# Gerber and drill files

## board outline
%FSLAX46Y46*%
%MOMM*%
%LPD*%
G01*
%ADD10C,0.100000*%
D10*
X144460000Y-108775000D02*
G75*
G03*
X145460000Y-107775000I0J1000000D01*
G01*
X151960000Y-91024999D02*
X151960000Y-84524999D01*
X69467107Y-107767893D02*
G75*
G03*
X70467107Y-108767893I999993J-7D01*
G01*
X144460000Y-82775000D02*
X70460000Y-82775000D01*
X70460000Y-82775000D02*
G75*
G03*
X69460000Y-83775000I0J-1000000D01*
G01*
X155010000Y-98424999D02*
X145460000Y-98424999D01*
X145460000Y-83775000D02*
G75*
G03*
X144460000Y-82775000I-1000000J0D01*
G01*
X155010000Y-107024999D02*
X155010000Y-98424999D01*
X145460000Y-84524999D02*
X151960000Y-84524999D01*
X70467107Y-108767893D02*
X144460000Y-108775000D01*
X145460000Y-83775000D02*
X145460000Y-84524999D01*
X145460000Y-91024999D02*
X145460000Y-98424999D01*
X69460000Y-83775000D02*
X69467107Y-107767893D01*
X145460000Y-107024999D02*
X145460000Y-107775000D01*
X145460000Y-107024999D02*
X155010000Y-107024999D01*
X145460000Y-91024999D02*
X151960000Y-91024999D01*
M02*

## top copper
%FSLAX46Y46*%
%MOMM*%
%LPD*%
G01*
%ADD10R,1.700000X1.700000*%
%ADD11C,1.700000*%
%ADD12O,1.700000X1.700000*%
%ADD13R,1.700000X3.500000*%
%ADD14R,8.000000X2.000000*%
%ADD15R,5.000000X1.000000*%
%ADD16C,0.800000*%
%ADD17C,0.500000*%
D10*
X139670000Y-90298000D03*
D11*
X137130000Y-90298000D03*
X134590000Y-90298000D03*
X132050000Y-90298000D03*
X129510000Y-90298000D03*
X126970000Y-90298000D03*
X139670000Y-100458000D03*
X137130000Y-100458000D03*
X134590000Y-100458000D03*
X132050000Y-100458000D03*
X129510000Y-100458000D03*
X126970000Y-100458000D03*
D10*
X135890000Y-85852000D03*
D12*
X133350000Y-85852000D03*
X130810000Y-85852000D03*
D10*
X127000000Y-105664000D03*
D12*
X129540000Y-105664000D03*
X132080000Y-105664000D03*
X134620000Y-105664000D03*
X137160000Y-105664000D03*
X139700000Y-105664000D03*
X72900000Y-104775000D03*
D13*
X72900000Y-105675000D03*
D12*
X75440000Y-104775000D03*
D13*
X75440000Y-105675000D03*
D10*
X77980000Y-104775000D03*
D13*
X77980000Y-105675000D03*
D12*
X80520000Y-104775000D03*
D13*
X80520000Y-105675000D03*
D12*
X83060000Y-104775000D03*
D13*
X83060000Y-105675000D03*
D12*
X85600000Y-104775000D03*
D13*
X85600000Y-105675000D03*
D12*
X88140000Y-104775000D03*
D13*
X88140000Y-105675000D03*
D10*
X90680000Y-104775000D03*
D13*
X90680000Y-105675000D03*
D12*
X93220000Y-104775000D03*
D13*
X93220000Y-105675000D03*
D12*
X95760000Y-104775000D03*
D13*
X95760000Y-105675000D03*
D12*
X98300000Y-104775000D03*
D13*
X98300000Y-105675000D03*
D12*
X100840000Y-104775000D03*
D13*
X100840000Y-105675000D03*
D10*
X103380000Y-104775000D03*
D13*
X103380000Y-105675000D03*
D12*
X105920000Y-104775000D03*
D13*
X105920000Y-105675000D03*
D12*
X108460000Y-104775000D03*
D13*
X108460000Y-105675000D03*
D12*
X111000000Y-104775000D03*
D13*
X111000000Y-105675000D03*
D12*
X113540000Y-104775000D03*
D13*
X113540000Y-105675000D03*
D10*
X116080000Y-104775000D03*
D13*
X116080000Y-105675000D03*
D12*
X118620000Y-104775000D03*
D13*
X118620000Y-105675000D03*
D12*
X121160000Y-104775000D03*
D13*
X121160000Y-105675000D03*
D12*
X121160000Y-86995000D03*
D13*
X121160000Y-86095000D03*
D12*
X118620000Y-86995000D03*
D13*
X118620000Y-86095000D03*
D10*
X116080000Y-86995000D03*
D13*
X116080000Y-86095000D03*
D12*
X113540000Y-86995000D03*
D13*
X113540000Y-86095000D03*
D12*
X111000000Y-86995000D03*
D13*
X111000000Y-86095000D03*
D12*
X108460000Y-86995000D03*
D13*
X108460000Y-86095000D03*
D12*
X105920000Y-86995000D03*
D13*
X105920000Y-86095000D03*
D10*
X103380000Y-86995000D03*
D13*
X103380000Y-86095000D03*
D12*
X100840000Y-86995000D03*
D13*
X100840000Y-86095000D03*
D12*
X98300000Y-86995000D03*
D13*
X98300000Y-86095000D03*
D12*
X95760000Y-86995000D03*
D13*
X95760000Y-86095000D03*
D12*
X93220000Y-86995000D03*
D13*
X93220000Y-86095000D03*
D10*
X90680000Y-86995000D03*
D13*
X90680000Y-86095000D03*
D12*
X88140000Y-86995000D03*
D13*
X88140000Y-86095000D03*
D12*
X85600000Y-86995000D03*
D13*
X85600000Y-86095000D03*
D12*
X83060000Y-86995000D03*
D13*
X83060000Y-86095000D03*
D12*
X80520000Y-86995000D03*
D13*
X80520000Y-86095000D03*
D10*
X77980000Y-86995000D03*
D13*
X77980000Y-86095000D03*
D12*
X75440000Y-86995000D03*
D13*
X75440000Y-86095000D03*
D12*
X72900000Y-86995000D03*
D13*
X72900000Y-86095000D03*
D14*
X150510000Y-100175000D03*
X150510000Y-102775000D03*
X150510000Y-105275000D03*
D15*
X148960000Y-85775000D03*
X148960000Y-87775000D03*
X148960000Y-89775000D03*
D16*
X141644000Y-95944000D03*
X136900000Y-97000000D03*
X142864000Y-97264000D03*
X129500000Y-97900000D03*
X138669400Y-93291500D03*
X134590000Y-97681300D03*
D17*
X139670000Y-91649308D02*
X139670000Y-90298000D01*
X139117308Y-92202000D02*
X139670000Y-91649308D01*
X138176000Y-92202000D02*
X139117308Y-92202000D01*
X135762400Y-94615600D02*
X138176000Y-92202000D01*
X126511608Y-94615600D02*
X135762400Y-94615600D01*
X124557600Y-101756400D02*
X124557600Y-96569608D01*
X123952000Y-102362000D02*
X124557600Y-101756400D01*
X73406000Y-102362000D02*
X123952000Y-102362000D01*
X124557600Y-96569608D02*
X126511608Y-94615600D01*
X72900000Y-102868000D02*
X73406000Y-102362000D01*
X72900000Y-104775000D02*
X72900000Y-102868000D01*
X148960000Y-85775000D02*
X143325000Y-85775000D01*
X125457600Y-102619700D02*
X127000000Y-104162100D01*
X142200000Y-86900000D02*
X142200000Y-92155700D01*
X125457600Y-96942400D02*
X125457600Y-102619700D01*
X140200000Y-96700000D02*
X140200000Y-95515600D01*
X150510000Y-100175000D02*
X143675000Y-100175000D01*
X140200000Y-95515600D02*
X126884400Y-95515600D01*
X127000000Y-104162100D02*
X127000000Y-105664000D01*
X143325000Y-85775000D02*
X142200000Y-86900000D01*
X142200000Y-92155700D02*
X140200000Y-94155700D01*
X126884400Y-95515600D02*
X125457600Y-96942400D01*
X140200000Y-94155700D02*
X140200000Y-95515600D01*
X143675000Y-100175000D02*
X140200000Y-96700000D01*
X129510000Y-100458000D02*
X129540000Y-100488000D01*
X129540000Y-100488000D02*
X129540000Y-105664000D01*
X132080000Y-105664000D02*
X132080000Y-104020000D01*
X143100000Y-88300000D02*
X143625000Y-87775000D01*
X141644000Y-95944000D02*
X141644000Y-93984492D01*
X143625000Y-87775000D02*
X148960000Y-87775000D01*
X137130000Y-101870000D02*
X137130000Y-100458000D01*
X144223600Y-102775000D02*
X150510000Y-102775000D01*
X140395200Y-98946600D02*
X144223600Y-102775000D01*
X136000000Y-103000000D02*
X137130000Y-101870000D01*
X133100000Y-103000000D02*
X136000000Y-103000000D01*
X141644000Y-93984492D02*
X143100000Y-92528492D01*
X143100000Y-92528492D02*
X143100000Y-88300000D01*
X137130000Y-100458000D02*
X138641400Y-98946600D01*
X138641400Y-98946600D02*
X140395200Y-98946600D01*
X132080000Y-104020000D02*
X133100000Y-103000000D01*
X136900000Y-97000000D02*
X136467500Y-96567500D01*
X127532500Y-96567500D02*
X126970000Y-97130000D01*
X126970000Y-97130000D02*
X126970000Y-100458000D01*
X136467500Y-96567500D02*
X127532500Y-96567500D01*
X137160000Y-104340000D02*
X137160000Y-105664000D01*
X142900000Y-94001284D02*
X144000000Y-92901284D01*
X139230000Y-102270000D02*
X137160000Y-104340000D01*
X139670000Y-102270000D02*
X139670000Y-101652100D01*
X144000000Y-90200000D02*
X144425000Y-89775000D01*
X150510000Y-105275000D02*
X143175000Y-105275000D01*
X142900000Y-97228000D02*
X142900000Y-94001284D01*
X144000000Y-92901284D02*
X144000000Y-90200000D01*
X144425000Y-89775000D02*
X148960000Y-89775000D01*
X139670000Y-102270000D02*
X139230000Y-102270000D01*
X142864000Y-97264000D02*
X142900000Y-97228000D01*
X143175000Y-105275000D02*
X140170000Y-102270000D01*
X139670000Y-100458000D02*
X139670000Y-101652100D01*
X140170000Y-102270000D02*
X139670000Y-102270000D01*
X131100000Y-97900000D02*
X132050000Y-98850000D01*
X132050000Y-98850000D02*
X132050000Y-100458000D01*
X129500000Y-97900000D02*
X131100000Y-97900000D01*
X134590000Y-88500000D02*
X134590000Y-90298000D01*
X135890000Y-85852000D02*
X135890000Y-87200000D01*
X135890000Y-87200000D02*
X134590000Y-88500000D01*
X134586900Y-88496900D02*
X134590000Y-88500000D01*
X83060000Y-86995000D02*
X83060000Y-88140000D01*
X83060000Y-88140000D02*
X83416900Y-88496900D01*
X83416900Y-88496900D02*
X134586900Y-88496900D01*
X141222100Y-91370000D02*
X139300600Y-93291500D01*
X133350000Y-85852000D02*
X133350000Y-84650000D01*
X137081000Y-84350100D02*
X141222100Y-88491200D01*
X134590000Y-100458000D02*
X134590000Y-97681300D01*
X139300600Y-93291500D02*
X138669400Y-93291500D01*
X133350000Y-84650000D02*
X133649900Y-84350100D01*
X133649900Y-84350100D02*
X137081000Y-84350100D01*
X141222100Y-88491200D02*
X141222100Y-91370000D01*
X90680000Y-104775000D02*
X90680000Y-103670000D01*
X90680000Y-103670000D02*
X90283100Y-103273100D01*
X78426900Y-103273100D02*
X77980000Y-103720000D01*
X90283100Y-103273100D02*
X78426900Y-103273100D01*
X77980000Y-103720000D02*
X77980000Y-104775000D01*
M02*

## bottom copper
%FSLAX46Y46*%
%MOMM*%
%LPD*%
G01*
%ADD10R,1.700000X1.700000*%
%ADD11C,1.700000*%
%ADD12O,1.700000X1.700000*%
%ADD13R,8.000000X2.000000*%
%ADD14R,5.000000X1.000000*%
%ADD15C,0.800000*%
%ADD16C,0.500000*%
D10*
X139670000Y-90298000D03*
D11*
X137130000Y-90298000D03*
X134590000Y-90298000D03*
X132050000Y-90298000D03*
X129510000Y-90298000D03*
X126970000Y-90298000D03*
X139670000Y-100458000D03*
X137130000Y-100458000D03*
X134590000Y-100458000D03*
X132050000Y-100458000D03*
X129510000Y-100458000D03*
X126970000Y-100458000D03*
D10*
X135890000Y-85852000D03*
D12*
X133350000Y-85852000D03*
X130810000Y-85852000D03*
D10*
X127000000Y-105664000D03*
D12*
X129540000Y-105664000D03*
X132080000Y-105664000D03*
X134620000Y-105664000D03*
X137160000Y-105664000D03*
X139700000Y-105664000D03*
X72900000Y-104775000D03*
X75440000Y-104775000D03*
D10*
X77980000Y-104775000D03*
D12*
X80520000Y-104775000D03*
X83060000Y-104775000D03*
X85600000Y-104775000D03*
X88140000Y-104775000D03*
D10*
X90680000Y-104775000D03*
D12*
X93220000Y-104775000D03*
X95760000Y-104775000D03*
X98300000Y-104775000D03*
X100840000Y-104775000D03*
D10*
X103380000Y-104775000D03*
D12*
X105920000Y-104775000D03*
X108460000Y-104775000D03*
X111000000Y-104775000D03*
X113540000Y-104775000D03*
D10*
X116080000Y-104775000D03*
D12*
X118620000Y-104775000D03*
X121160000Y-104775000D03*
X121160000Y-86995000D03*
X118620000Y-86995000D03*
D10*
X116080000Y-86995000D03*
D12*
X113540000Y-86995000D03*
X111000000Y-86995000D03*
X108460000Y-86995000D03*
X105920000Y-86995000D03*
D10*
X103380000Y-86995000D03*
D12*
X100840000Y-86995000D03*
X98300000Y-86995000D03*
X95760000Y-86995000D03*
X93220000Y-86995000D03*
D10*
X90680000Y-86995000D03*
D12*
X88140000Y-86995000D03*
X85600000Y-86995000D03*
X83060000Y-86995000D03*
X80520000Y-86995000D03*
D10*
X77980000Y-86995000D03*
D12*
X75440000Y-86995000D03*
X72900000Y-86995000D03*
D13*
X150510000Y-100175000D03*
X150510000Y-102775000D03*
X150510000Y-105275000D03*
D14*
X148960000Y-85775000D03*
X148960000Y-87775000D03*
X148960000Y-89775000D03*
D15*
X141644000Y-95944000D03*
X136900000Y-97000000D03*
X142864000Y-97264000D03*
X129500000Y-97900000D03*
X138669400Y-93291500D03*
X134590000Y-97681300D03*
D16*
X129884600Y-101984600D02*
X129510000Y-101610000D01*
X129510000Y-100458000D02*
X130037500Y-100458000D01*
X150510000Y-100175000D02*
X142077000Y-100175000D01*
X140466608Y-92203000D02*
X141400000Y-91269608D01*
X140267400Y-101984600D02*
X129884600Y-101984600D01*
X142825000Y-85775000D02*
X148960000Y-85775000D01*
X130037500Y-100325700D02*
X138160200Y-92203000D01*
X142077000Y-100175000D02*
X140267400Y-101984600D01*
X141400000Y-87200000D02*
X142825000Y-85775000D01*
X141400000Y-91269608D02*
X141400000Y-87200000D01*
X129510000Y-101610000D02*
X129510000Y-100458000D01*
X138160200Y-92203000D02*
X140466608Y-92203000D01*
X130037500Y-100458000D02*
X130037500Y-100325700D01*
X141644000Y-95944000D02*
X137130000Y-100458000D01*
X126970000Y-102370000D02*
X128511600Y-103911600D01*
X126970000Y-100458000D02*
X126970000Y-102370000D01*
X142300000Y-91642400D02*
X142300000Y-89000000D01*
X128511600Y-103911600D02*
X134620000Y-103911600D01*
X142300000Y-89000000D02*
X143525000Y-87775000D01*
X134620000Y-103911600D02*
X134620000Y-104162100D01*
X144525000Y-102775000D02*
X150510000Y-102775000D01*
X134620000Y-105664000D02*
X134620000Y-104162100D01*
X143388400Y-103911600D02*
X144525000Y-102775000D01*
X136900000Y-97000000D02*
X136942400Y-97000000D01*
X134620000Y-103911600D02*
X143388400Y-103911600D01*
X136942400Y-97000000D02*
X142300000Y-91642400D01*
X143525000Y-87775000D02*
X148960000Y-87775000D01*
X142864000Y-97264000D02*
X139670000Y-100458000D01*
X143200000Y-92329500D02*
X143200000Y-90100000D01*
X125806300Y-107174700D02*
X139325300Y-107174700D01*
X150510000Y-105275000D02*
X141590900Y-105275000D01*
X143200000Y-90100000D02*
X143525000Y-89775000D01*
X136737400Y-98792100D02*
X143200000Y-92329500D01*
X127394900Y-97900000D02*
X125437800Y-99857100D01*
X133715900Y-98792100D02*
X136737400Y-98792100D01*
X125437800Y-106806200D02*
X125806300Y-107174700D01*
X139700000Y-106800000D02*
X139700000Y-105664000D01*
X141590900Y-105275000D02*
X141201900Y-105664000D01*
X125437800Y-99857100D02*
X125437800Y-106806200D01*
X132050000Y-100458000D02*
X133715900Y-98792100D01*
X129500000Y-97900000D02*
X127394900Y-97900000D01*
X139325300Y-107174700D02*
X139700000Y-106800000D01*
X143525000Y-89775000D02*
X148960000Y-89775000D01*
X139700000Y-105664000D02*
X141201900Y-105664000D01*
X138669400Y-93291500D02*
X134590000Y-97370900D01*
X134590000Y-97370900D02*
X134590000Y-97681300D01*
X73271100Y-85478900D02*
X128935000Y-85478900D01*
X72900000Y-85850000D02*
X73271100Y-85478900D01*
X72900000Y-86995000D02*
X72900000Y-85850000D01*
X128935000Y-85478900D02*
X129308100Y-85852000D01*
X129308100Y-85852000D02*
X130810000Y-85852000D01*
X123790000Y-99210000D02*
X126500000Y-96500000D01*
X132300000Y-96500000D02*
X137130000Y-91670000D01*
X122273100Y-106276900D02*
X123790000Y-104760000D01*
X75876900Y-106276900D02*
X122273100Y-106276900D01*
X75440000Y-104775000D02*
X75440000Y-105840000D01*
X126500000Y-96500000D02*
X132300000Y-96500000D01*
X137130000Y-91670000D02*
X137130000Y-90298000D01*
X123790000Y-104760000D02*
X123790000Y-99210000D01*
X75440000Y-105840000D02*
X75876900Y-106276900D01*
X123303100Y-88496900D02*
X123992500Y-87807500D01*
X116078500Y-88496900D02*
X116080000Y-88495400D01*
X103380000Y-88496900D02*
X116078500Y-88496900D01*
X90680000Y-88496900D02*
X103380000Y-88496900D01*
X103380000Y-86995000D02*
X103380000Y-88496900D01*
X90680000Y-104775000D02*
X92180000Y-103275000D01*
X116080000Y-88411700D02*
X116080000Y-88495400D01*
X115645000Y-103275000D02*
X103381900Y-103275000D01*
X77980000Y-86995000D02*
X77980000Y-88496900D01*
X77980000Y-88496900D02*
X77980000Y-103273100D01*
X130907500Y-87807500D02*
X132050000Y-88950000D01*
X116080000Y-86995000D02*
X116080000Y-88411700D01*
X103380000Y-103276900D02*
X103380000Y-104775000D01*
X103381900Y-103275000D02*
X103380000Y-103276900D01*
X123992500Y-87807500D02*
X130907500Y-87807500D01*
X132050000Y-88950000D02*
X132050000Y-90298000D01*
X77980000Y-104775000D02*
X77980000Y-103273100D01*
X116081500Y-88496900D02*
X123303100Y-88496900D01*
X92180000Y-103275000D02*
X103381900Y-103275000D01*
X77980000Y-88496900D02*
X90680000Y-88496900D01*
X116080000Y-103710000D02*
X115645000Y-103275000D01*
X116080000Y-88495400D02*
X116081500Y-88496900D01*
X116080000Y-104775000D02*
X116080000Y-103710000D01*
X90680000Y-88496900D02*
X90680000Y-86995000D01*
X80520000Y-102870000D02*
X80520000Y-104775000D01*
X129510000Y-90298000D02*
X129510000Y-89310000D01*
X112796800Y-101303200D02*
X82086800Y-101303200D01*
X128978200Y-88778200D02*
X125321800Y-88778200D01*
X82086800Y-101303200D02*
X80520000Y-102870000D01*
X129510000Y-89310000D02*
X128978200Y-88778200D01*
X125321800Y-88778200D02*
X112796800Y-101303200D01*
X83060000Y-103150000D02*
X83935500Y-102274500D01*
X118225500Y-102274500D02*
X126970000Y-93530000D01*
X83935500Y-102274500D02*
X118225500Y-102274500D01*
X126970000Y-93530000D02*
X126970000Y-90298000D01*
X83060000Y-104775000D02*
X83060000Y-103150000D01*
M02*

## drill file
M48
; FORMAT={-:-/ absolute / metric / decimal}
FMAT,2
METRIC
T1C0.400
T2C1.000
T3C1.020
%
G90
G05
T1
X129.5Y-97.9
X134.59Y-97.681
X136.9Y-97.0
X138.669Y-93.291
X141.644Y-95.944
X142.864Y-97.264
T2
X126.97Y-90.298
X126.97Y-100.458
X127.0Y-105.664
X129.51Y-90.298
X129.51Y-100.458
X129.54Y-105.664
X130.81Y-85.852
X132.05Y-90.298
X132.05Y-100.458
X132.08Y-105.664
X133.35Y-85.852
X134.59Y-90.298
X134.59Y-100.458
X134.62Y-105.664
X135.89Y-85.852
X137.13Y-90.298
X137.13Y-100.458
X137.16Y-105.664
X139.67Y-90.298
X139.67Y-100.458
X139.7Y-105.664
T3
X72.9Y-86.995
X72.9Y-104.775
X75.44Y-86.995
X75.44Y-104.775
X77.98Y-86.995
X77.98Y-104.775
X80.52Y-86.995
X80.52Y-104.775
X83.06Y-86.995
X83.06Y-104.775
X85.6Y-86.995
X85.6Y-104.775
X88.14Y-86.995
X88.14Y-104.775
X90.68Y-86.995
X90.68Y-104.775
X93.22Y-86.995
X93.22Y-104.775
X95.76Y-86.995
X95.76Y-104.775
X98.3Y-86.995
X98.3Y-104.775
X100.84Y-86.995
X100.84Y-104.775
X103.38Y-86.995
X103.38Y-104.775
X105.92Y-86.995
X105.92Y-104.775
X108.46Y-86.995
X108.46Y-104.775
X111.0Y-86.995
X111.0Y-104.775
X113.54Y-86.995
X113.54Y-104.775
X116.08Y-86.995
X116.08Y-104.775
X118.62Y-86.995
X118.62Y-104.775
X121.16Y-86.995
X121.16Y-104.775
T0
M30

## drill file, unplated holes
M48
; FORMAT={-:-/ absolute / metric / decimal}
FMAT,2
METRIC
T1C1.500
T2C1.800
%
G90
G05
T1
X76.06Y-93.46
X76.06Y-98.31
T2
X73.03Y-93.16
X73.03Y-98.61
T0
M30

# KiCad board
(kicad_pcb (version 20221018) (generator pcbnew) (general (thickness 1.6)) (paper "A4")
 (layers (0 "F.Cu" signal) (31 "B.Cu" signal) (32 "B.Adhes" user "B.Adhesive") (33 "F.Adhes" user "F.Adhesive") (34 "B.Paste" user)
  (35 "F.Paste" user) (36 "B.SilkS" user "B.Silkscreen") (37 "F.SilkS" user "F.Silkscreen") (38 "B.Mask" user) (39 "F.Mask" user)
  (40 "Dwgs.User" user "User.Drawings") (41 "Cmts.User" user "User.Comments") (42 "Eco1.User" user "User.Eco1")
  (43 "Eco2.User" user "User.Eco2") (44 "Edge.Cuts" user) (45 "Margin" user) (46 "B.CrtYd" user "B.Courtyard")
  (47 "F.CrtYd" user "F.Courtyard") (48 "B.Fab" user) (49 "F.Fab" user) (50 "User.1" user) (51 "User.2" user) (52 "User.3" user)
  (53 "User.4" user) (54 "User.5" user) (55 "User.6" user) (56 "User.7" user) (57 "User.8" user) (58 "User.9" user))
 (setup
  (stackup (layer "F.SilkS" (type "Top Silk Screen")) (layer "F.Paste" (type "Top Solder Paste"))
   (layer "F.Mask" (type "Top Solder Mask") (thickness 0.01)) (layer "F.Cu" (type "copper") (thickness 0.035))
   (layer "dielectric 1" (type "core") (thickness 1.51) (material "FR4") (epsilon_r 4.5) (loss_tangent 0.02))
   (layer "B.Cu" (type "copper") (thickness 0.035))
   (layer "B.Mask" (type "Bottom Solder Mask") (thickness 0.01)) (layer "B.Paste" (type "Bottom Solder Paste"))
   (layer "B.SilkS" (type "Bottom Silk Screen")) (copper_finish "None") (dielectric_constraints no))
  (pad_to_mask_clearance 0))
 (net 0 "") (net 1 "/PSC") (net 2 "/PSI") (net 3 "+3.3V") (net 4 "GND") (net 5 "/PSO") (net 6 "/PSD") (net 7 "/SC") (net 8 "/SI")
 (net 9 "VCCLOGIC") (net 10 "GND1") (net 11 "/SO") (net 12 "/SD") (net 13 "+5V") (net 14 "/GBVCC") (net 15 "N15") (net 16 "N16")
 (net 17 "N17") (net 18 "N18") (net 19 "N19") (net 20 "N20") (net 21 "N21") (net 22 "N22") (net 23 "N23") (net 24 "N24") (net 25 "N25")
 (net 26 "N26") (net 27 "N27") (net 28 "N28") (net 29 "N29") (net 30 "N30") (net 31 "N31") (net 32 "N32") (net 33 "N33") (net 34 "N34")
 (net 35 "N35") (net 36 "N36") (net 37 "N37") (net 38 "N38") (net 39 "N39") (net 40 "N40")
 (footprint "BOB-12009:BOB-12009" (layer "F.Cu") (at 133.35 95.758 -90)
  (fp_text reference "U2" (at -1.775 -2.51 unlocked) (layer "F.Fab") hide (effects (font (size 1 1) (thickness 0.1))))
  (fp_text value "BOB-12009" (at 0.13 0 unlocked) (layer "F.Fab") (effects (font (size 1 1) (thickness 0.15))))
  (pad "1" thru_hole rect (at -5.46 -6.32 270) (size 1.7 1.7) (drill 1) (layers "*.Cu" "*.Mask") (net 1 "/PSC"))
  (pad "2" thru_hole circle (at -5.46 -3.78 270) (size 1.7 1.7) (drill 1) (layers "*.Cu" "*.Mask") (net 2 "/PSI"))
  (pad "3" thru_hole circle (at -5.46 -1.24 270) (size 1.7 1.7) (drill 1) (layers "*.Cu" "*.Mask") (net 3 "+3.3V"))
  (pad "4" thru_hole circle (at -5.46 1.3 270) (size 1.7 1.7) (drill 1) (layers "*.Cu" "*.Mask") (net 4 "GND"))
  (pad "5" thru_hole circle (at -5.46 3.84 270) (size 1.7 1.7) (drill 1) (layers "*.Cu" "*.Mask") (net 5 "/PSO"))
  (pad "6" thru_hole circle (at -5.46 6.38 270) (size 1.7 1.7) (drill 1) (layers "*.Cu" "*.Mask") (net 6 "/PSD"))
  (pad "7" thru_hole circle (at 4.7 -6.32 270) (size 1.7 1.7) (drill 1) (layers "*.Cu" "*.Mask") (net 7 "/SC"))
  (pad "8" thru_hole circle (at 4.7 -3.78 270) (size 1.7 1.7) (drill 1) (layers "*.Cu" "*.Mask") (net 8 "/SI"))
  (pad "9" thru_hole circle (at 4.7 -1.24 270) (size 1.7 1.7) (drill 1) (layers "*.Cu" "*.Mask") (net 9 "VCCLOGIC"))
  (pad "10" thru_hole circle (at 4.7 1.3 270) (size 1.7 1.7) (drill 1) (layers "*.Cu" "*.Mask") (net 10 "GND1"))
  (pad "11" thru_hole circle (at 4.7 3.84 270) (size 1.7 1.7) (drill 1) (layers "*.Cu" "*.Mask") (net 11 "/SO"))
  (pad "12" thru_hole circle (at 4.7 6.38 270) (size 1.7 1.7) (drill 1) (layers "*.Cu" "*.Mask") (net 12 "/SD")))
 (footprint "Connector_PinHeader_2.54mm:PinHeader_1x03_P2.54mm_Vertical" (layer "F.Cu") (at 135.89 85.852 -90)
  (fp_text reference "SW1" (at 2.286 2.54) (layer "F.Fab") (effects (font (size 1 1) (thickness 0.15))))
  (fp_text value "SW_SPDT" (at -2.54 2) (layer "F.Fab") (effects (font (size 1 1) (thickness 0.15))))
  (pad "1" thru_hole rect (at 0 0 270) (size 1.7 1.7) (drill 1) (layers "*.Cu" "*.Mask") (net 3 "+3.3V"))
  (pad "2" thru_hole oval (at 0 2.54 270) (size 1.7 1.7) (drill 1) (layers "*.Cu" "*.Mask") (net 9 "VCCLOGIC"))
  (pad "3" thru_hole oval (at 0 5.08 270) (size 1.7 1.7) (drill 1) (layers "*.Cu" "*.Mask") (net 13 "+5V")))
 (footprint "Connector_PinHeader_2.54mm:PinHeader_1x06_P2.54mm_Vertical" (layer "F.Cu") (at 127 105.664 90)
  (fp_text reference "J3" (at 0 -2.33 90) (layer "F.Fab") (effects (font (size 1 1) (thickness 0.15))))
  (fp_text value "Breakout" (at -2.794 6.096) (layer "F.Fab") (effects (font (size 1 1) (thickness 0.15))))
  (pad "1" thru_hole rect (at 0 0 90) (size 1.7 1.7) (drill 1) (layers "*.Cu" "*.Mask") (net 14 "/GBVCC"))
  (pad "2" thru_hole oval (at 0 2.54 90) (size 1.7 1.7) (drill 1) (layers "*.Cu" "*.Mask") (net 11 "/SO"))
  (pad "3" thru_hole oval (at 0 5.08 90) (size 1.7 1.7) (drill 1) (layers "*.Cu" "*.Mask") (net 8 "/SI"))
  (pad "4" thru_hole oval (at 0 7.62 90) (size 1.7 1.7) (drill 1) (layers "*.Cu" "*.Mask") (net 12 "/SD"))
  (pad "5" thru_hole oval (at 0 10.16 90) (size 1.7 1.7) (drill 1) (layers "*.Cu" "*.Mask") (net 7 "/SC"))
  (pad "6" thru_hole oval (at 0 12.7 90) (size 1.7 1.7) (drill 1) (layers "*.Cu" "*.Mask") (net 10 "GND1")))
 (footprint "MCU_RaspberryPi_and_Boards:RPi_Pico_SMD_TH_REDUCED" (layer "F.Cu") (at 97.03 95.885 90)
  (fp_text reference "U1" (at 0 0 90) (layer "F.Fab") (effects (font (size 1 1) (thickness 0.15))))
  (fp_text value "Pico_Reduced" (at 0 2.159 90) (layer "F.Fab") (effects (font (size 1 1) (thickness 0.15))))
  (pad "" np_thru_hole oval (at -2.725 -24 90) (size 1.8 1.8) (drill 1.8) (layers "*.Cu" "*.Mask"))
  (pad "" np_thru_hole oval (at -2.425 -20.97 90) (size 1.5 1.5) (drill 1.5) (layers "*.Cu" "*.Mask"))
  (pad "" np_thru_hole oval (at 2.425 -20.97 90) (size 1.5 1.5) (drill 1.5) (layers "*.Cu" "*.Mask"))
  (pad "" np_thru_hole oval (at 2.725 -24 90) (size 1.8 1.8) (drill 1.8) (layers "*.Cu" "*.Mask"))
  (pad "1" thru_hole oval (at -8.89 -24.13 90) (size 1.7 1.7) (drill 1.02) (layers "*.Cu" "*.Mask") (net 1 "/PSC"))
  (pad "1" smd rect (at -8.89 -24.13 90) (size 3.5 1.7) (drill (offset -0.9 0)) (layers "F.Cu" "F.Mask") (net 1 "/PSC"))
  (pad "2" thru_hole oval (at -8.89 -21.59 90) (size 1.7 1.7) (drill 1.02) (layers "*.Cu" "*.Mask") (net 2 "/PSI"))
  (pad "2" smd rect (at -8.89 -21.59 90) (size 3.5 1.7) (drill (offset -0.9 0)) (layers "F.Cu" "F.Mask") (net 2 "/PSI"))
  (pad "3" thru_hole rect (at -8.89 -19.05 90) (size 1.7 1.7) (drill 1.02) (layers "*.Cu" "*.Mask") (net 4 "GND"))
  (pad "3" smd rect (at -8.89 -19.05 90) (size 3.5 1.7) (drill (offset -0.9 0)) (layers "F.Cu" "F.Mask") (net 4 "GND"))
  (pad "4" thru_hole oval (at -8.89 -16.51 90) (size 1.7 1.7) (drill 1.02) (layers "*.Cu" "*.Mask") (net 5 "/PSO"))
  (pad "4" smd rect (at -8.89 -16.51 90) (size 3.5 1.7) (drill (offset -0.9 0)) (layers "F.Cu" "F.Mask") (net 5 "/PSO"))
  (pad "5" thru_hole oval (at -8.89 -13.97 90) (size 1.7 1.7) (drill 1.02) (layers "*.Cu" "*.Mask") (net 6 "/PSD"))
  (pad "5" smd rect (at -8.89 -13.97 90) (size 3.5 1.7) (drill (offset -0.9 0)) (layers "F.Cu" "F.Mask") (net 6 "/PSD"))
  (pad "6" thru_hole oval (at -8.89 -11.43 90) (size 1.7 1.7) (drill 1.02) (layers "*.Cu" "*.Mask") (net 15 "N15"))
  (pad "6" smd rect (at -8.89 -11.43 90) (size 3.5 1.7) (drill (offset -0.9 0)) (layers "F.Cu" "F.Mask") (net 15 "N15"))
  (pad "7" thru_hole oval (at -8.89 -8.89 90) (size 1.7 1.7) (drill 1.02) (layers "*.Cu" "*.Mask") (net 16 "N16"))
  (pad "7" smd rect (at -8.89 -8.89 90) (size 3.5 1.7) (drill (offset -0.9 0)) (layers "F.Cu" "F.Mask") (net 16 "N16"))
  (pad "8" thru_hole rect (at -8.89 -6.35 90) (size 1.7 1.7) (drill 1.02) (layers "*.Cu" "*.Mask") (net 4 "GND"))
  (pad "8" smd rect (at -8.89 -6.35 90) (size 3.5 1.7) (drill (offset -0.9 0)) (layers "F.Cu" "F.Mask") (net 4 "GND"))
  (pad "9" thru_hole oval (at -8.89 -3.81 90) (size 1.7 1.7) (drill 1.02) (layers "*.Cu" "*.Mask") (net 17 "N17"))
  (pad "9" smd rect (at -8.89 -3.81 90) (size 3.5 1.7) (drill (offset -0.9 0)) (layers "F.Cu" "F.Mask") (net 17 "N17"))
  (pad "10" thru_hole oval (at -8.89 -1.27 90) (size 1.7 1.7) (drill 1.02) (layers "*.Cu" "*.Mask") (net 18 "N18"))
  (pad "10" smd rect (at -8.89 -1.27 90) (size 3.5 1.7) (drill (offset -0.9 0)) (layers "F.Cu" "F.Mask") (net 18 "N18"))
  (pad "11" thru_hole oval (at -8.89 1.27 90) (size 1.7 1.7) (drill 1.02) (layers "*.Cu" "*.Mask") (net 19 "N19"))
  (pad "11" smd rect (at -8.89 1.27 90) (size 3.5 1.7) (drill (offset -0.9 0)) (layers "F.Cu" "F.Mask") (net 19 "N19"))
  (pad "12" thru_hole oval (at -8.89 3.81 90) (size 1.7 1.7) (drill 1.02) (layers "*.Cu" "*.Mask") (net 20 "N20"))
  (pad "12" smd rect (at -8.89 3.81 90) (size 3.5 1.7) (drill (offset -0.9 0)) (layers "F.Cu" "F.Mask") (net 20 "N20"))
  (pad "13" thru_hole rect (at -8.89 6.35 90) (size 1.7 1.7) (drill 1.02) (layers "*.Cu" "*.Mask") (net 4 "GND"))
  (pad "13" smd rect (at -8.89 6.35 90) (size 3.5 1.7) (drill (offset -0.9 0)) (layers "F.Cu" "F.Mask") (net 4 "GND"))
  (pad "14" thru_hole oval (at -8.89 8.89 90) (size 1.7 1.7) (drill 1.02) (layers "*.Cu" "*.Mask") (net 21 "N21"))
  (pad "14" smd rect (at -8.89 8.89 90) (size 3.5 1.7) (drill (offset -0.9 0)) (layers "F.Cu" "F.Mask") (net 21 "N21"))
  (pad "15" thru_hole oval (at -8.89 11.43 90) (size 1.7 1.7) (drill 1.02) (layers "*.Cu" "*.Mask") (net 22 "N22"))
  (pad "15" smd rect (at -8.89 11.43 90) (size 3.5 1.7) (drill (offset -0.9 0)) (layers "F.Cu" "F.Mask") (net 22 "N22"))
  (pad "16" thru_hole oval (at -8.89 13.97 90) (size 1.7 1.7) (drill 1.02) (layers "*.Cu" "*.Mask") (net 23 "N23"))
  (pad "16" smd rect (at -8.89 13.97 90) (size 3.5 1.7) (drill (offset -0.9 0)) (layers "F.Cu" "F.Mask") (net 23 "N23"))
  (pad "17" thru_hole oval (at -8.89 16.51 90) (size 1.7 1.7) (drill 1.02) (layers "*.Cu" "*.Mask") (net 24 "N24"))
  (pad "17" smd rect (at -8.89 16.51 90) (size 3.5 1.7) (drill (offset -0.9 0)) (layers "F.Cu" "F.Mask") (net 24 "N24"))
  (pad "18" thru_hole rect (at -8.89 19.05 90) (size 1.7 1.7) (drill 1.02) (layers "*.Cu" "*.Mask") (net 4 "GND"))
  (pad "18" smd rect (at -8.89 19.05 90) (size 3.5 1.7) (drill (offset -0.9 0)) (layers "F.Cu" "F.Mask") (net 4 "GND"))
  (pad "19" thru_hole oval (at -8.89 21.59 90) (size 1.7 1.7) (drill 1.02) (layers "*.Cu" "*.Mask") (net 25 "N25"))
  (pad "19" smd rect (at -8.89 21.59 90) (size 3.5 1.7) (drill (offset -0.9 0)) (layers "F.Cu" "F.Mask") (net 25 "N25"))
  (pad "20" thru_hole oval (at -8.89 24.13 90) (size 1.7 1.7) (drill 1.02) (layers "*.Cu" "*.Mask") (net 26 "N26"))
  (pad "20" smd rect (at -8.89 24.13 90) (size 3.5 1.7) (drill (offset -0.9 0)) (layers "F.Cu" "F.Mask") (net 26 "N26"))
  (pad "21" thru_hole oval (at 8.89 24.13 90) (size 1.7 1.7) (drill 1.02) (layers "*.Cu" "*.Mask") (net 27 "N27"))
  (pad "21" smd rect (at 8.89 24.13 90) (size 3.5 1.7) (drill (offset 0.9 0)) (layers "F.Cu" "F.Mask") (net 27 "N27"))
  (pad "22" thru_hole oval (at 8.89 21.59 90) (size 1.7 1.7) (drill 1.02) (layers "*.Cu" "*.Mask") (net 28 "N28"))
  (pad "22" smd rect (at 8.89 21.59 90) (size 3.5 1.7) (drill (offset 0.9 0)) (layers "F.Cu" "F.Mask") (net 28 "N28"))
  (pad "23" thru_hole rect (at 8.89 19.05 90) (size 1.7 1.7) (drill 1.02) (layers "*.Cu" "*.Mask") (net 4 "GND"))
  (pad "23" smd rect (at 8.89 19.05 90) (size 3.5 1.7) (drill (offset 0.9 0)) (layers "F.Cu" "F.Mask") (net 4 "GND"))
  (pad "24" thru_hole oval (at 8.89 16.51 90) (size 1.7 1.7) (drill 1.02) (layers "*.Cu" "*.Mask") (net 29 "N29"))
  (pad "24" smd rect (at 8.89 16.51 90) (size 3.5 1.7) (drill (offset 0.9 0)) (layers "F.Cu" "F.Mask") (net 29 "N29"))
  (pad "25" thru_hole oval (at 8.89 13.97 90) (size 1.7 1.7) (drill 1.02) (layers "*.Cu" "*.Mask") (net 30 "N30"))
  (pad "25" smd rect (at 8.89 13.97 90) (size 3.5 1.7) (drill (offset 0.9 0)) (layers "F.Cu" "F.Mask") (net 30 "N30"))
  (pad "26" thru_hole oval (at 8.89 11.43 90) (size 1.7 1.7) (drill 1.02) (layers "*.Cu" "*.Mask") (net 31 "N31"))
  (pad "26" smd rect (at 8.89 11.43 90) (size 3.5 1.7) (drill (offset 0.9 0)) (layers "F.Cu" "F.Mask") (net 31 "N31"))
  (pad "27" thru_hole oval (at 8.89 8.89 90) (size 1.7 1.7) (drill 1.02) (layers "*.Cu" "*.Mask") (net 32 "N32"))
  (pad "27" smd rect (at 8.89 8.89 90) (size 3.5 1.7) (drill (offset 0.9 0)) (layers "F.Cu" "F.Mask") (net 32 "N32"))
  (pad "28" thru_hole rect (at 8.89 6.35 90) (size 1.7 1.7) (drill 1.02) (layers "*.Cu" "*.Mask") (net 4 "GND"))
  (pad "28" smd rect (at 8.89 6.35 90) (size 3.5 1.7) (drill (offset 0.9 0)) (layers "F.Cu" "F.Mask") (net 4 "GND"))
  (pad "29" thru_hole oval (at 8.89 3.81 90) (size 1.7 1.7) (drill 1.02) (layers "*.Cu" "*.Mask") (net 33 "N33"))
  (pad "29" smd rect (at 8.89 3.81 90) (size 3.5 1.7) (drill (offset 0.9 0)) (layers "F.Cu" "F.Mask") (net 33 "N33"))
  (pad "30" thru_hole oval (at 8.89 1.27 90) (size 1.7 1.7) (drill 1.02) (layers "*.Cu" "*.Mask") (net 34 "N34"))
  (pad "30" smd rect (at 8.89 1.27 90) (size 3.5 1.7) (drill (offset 0.9 0)) (layers "F.Cu" "F.Mask") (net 34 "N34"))
  (pad "31" thru_hole oval (at 8.89 -1.27 90) (size 1.7 1.7) (drill 1.02) (layers "*.Cu" "*.Mask") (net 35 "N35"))
  (pad "31" smd rect (at 8.89 -1.27 90) (size 3.5 1.7) (drill (offset 0.9 0)) (layers "F.Cu" "F.Mask") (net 35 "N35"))
  (pad "32" thru_hole oval (at 8.89 -3.81 90) (size 1.7 1.7) (drill 1.02) (layers "*.Cu" "*.Mask") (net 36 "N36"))
  (pad "32" smd rect (at 8.89 -3.81 90) (size 3.5 1.7) (drill (offset 0.9 0)) (layers "F.Cu" "F.Mask") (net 36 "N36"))
  (pad "33" thru_hole rect (at 8.89 -6.35 90) (size 1.7 1.7) (drill 1.02) (layers "*.Cu" "*.Mask") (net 4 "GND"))
  (pad "33" smd rect (at 8.89 -6.35 90) (size 3.5 1.7) (drill (offset 0.9 0)) (layers "F.Cu" "F.Mask") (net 4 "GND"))
  (pad "34" thru_hole oval (at 8.89 -8.89 90) (size 1.7 1.7) (drill 1.02) (layers "*.Cu" "*.Mask") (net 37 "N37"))
  (pad "34" smd rect (at 8.89 -8.89 90) (size 3.5 1.7) (drill (offset 0.9 0)) (layers "F.Cu" "F.Mask") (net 37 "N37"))
  (pad "35" thru_hole oval (at 8.89 -11.43 90) (size 1.7 1.7) (drill 1.02) (layers "*.Cu" "*.Mask") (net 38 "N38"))
  (pad "35" smd rect (at 8.89 -11.43 90) (size 3.5 1.7) (drill (offset 0.9 0)) (layers "F.Cu" "F.Mask") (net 38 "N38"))
  (pad "36" thru_hole oval (at 8.89 -13.97 90) (size 1.7 1.7) (drill 1.02) (layers "*.Cu" "*.Mask") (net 3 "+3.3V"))
  (pad "36" smd rect (at 8.89 -13.97 90) (size 3.5 1.7) (drill (offset 0.9 0)) (layers "F.Cu" "F.Mask") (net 3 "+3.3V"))
  (pad "37" thru_hole oval (at 8.89 -16.51 90) (size 1.7 1.7) (drill 1.02) (layers "*.Cu" "*.Mask") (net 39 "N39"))
  (pad "37" smd rect (at 8.89 -16.51 90) (size 3.5 1.7) (drill (offset 0.9 0)) (layers "F.Cu" "F.Mask") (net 39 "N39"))
  (pad "38" thru_hole rect (at 8.89 -19.05 90) (size 1.7 1.7) (drill 1.02) (layers "*.Cu" "*.Mask") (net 4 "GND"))
  (pad "38" smd rect (at 8.89 -19.05 90) (size 3.5 1.7) (drill (offset 0.9 0)) (layers "F.Cu" "F.Mask") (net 4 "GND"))
  (pad "39" thru_hole oval (at 8.89 -21.59 90) (size 1.7 1.7) (drill 1.02) (layers "*.Cu" "*.Mask") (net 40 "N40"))
  (pad "39" smd rect (at 8.89 -21.59 90) (size 3.5 1.7) (drill (offset 0.9 0)) (layers "F.Cu" "F.Mask") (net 40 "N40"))
  (pad "40" thru_hole oval (at 8.89 -24.13 90) (size 1.7 1.7) (drill 1.02) (layers "*.Cu" "*.Mask") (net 13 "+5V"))
  (pad "40" smd rect (at 8.89 -24.13 90) (size 3.5 1.7) (drill (offset 0.9 0)) (layers "F.Cu" "F.Mask") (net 13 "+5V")))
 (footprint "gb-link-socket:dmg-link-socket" (layer "B.Cu") (at 150.51 102.775 -90)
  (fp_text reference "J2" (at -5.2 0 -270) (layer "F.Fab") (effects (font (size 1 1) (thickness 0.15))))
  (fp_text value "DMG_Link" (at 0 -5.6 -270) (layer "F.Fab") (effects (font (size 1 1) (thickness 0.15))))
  (pad "1" connect rect (at -2.6 0 270) (size 2 8) (layers "F.Cu" "F.Mask") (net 14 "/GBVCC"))
  (pad "2" connect rect (at -2.6 0 270) (size 2 8) (layers "B.Cu" "B.Mask") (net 11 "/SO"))
  (pad "3" connect rect (at 0 0 270) (size 2 8) (layers "F.Cu" "F.Mask") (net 8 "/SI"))
  (pad "4" connect rect (at 0 0 270) (size 2 8) (layers "B.Cu" "B.Mask") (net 12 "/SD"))
  (pad "5" connect rect (at 2.5 0 270) (size 2 8) (layers "F.Cu" "F.Mask") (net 7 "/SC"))
  (pad "6" connect rect (at 2.5 0 270) (size 2 8) (layers "B.Cu" "B.Mask") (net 10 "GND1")))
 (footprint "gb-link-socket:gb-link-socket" (layer "B.Cu") (at 148.96 87.775 -90)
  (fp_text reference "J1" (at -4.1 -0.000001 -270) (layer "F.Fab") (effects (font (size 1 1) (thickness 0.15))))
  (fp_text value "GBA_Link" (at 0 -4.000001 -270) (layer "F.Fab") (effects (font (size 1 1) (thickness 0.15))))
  (pad "1" connect rect (at -2 0 270) (size 1 5) (layers "F.Cu" "F.Mask") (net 14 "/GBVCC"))
  (pad "2" connect rect (at -2 0 270) (size 1 5) (layers "B.Cu" "B.Mask") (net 11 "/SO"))
  (pad "3" connect rect (at 0 0 270) (size 1 5) (layers "F.Cu" "F.Mask") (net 8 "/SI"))
  (pad "4" connect rect (at 0 0 270) (size 1 5) (layers "B.Cu" "B.Mask") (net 12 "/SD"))
  (pad "5" connect rect (at 2 0 270) (size 1 5) (layers "F.Cu" "F.Mask") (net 7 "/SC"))
  (pad "6" connect rect (at 2 0 270) (size 1 5) (layers "B.Cu" "B.Mask") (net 10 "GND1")))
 (gr_arc (start 145.46 107.775) (mid 145.167107 108.482107) (end 144.46 108.775) (stroke (width 0.1) (type default)) (layer "Edge.Cuts"))
 (gr_line (start 151.96 91.024999) (end 151.96 84.524999) (stroke (width 0.1) (type default)) (layer "Edge.Cuts"))
 (gr_arc (start 70.467107 108.767893) (mid 69.759998 108.475002) (end 69.467107 107.767893) (stroke (width 0.1) (type default))
  (layer "Edge.Cuts"))
 (gr_line (start 144.46 82.775) (end 70.46 82.775) (stroke (width 0.1) (type default)) (layer "Edge.Cuts"))
 (gr_arc (start 69.46 83.775) (mid 69.752893 83.067893) (end 70.46 82.775) (stroke (width 0.1) (type default)) (layer "Edge.Cuts"))
 (gr_line (start 155.01 98.424999) (end 145.46 98.424999) (stroke (width 0.1) (type default)) (layer "Edge.Cuts"))
 (gr_arc (start 144.46 82.775) (mid 145.167107 83.067893) (end 145.46 83.775) (stroke (width 0.1) (type default)) (layer "Edge.Cuts"))
 (gr_line (start 155.01 107.024999) (end 155.01 98.424999) (stroke (width 0.1) (type default)) (layer "Edge.Cuts"))
 (gr_line (start 145.46 84.524999) (end 151.96 84.524999) (stroke (width 0.1) (type default)) (layer "Edge.Cuts"))
 (gr_line (start 70.467107 108.767893) (end 144.46 108.775) (stroke (width 0.1) (type default)) (layer "Edge.Cuts"))
 (gr_line (start 145.46 83.775) (end 145.46 84.524999) (stroke (width 0.1) (type default)) (layer "Edge.Cuts"))
 (gr_line (start 145.46 91.024999) (end 145.46 98.424999) (stroke (width 0.1) (type default)) (layer "Edge.Cuts"))
 (gr_line (start 69.46 83.775) (end 69.467107 107.767893) (stroke (width 0.1) (type default)) (layer "Edge.Cuts"))
 (gr_line (start 145.46 107.024999) (end 145.46 107.775) (stroke (width 0.1) (type default)) (layer "Edge.Cuts"))
 (gr_line (start 145.46 107.024999) (end 155.01 107.024999) (stroke (width 0.1) (type default)) (layer "Edge.Cuts"))
 (gr_line (start 145.46 91.024999) (end 151.96 91.024999) (stroke (width 0.1) (type default)) (layer "Edge.Cuts"))
 (segment (start 148.96 85.775) (end 143.325 85.775) (width 0.5) (layer "F.Cu") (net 14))
 (segment (start 125.4576 102.6197) (end 127 104.1621) (width 0.5) (layer "F.Cu") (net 14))
 (segment (start 142.2 86.9) (end 142.2 92.1557) (width 0.5) (layer "F.Cu") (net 14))
 (segment (start 125.4576 96.9424) (end 125.4576 102.6197) (width 0.5) (layer "F.Cu") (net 14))
 (segment (start 140.2 96.7) (end 140.2 95.5156) (width 0.5) (layer "F.Cu") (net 14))
 (segment (start 150.51 100.175) (end 143.675 100.175) (width 0.5) (layer "F.Cu") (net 14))
 (segment (start 140.2 95.5156) (end 126.8844 95.5156) (width 0.5) (layer "F.Cu") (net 14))
 (segment (start 127 104.1621) (end 127 105.664) (width 0.5) (layer "F.Cu") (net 14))
 (segment (start 143.325 85.775) (end 142.2 86.9) (width 0.5) (layer "F.Cu") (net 14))
 (segment (start 142.2 92.1557) (end 140.2 94.1557) (width 0.5) (layer "F.Cu") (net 14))
 (segment (start 126.8844 95.5156) (end 125.4576 96.9424) (width 0.5) (layer "F.Cu") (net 14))
 (segment (start 140.2 94.1557) (end 140.2 95.5156) (width 0.5) (layer "F.Cu") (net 14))
 (segment (start 143.675 100.175) (end 140.2 96.7) (width 0.5) (layer "F.Cu") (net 14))
 (segment (start 129.51 100.458) (end 129.54 100.488) (width 0.5) (layer "F.Cu") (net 11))
 (segment (start 129.54 100.488) (end 129.54 105.664) (width 0.5) (layer "F.Cu") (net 11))
 (segment (start 129.8846 101.9846) (end 129.51 101.61) (width 0.5) (layer "B.Cu") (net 11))
 (segment (start 129.51 100.458) (end 130.0375 100.458) (width 0.5) (layer "B.Cu") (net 11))
 (segment (start 150.51 100.175) (end 142.077 100.175) (width 0.5) (layer "B.Cu") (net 11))
 (segment (start 140.466608 92.203) (end 141.4 91.269608) (width 0.5) (layer "B.Cu") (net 11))
 (segment (start 140.2674 101.9846) (end 129.8846 101.9846) (width 0.5) (layer "B.Cu") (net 11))
 (segment (start 142.825 85.775) (end 148.96 85.775) (width 0.5) (layer "B.Cu") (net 11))
 (segment (start 130.0375 100.3257) (end 138.1602 92.203) (width 0.5) (layer "B.Cu") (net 11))
 (segment (start 142.077 100.175) (end 140.2674 101.9846) (width 0.5) (layer "B.Cu") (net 11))
 (segment (start 141.4 87.2) (end 142.825 85.775) (width 0.5) (layer "B.Cu") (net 11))
 (segment (start 141.4 91.269608) (end 141.4 87.2) (width 0.5) (layer "B.Cu") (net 11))
 (segment (start 129.51 101.61) (end 129.51 100.458) (width 0.5) (layer "B.Cu") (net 11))
 (segment (start 138.1602 92.203) (end 140.466608 92.203) (width 0.5) (layer "B.Cu") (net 11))
 (segment (start 130.0375 100.458) (end 130.0375 100.3257) (width 0.5) (layer "B.Cu") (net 11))
 (segment (start 132.08 105.664) (end 132.08 104.02) (width 0.5) (layer "F.Cu") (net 8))
 (segment (start 143.1 88.3) (end 143.625 87.775) (width 0.5) (layer "F.Cu") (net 8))
 (segment (start 141.644 95.944) (end 141.644 93.984492) (width 0.5) (layer "F.Cu") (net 8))
 (segment (start 143.625 87.775) (end 148.96 87.775) (width 0.5) (layer "F.Cu") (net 8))
 (segment (start 137.13 101.87) (end 137.13 100.458) (width 0.5) (layer "F.Cu") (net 8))
 (segment (start 144.2236 102.775) (end 150.51 102.775) (width 0.5) (layer "F.Cu") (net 8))
 (segment (start 140.3952 98.9466) (end 144.2236 102.775) (width 0.5) (layer "F.Cu") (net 8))
 (segment (start 136 103) (end 137.13 101.87) (width 0.5) (layer "F.Cu") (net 8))
 (segment (start 133.1 103) (end 136 103) (width 0.5) (layer "F.Cu") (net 8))
 (segment (start 141.644 93.984492) (end 143.1 92.528492) (width 0.5) (layer "F.Cu") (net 8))
 (segment (start 143.1 92.528492) (end 143.1 88.3) (width 0.5) (layer "F.Cu") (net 8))
 (segment (start 137.13 100.458) (end 138.6414 98.9466) (width 0.5) (layer "F.Cu") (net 8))
 (segment (start 138.6414 98.9466) (end 140.3952 98.9466) (width 0.5) (layer "F.Cu") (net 8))
 (segment (start 132.08 104.02) (end 133.1 103) (width 0.5) (layer "F.Cu") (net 8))
 (via (at 141.644 95.944) (size 0.8) (drill 0.4) (layers "F.Cu" "B.Cu") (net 8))
 (segment (start 141.644 95.944) (end 137.13 100.458) (width 0.5) (layer "B.Cu") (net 8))
 (segment (start 136.9 97) (end 136.4675 96.5675) (width 0.5) (layer "F.Cu") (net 12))
 (segment (start 127.5325 96.5675) (end 126.97 97.13) (width 0.5) (layer "F.Cu") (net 12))
 (segment (start 126.97 97.13) (end 126.97 100.458) (width 0.5) (layer "F.Cu") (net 12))
 (segment (start 136.4675 96.5675) (end 127.5325 96.5675) (width 0.5) (layer "F.Cu") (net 12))
 (via (at 136.9 97) (size 0.8) (drill 0.4) (layers "F.Cu" "B.Cu") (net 12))
 (segment (start 126.97 102.37) (end 128.5116 103.9116) (width 0.5) (layer "B.Cu") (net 12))
 (segment (start 126.97 100.458) (end 126.97 102.37) (width 0.5) (layer "B.Cu") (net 12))
 (segment (start 142.3 91.6424) (end 142.3 89) (width 0.5) (layer "B.Cu") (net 12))
 (segment (start 128.5116 103.9116) (end 134.62 103.9116) (width 0.5) (layer "B.Cu") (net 12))
 (segment (start 142.3 89) (end 143.525 87.775) (width 0.5) (layer "B.Cu") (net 12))
 (segment (start 134.62 103.9116) (end 134.62 104.1621) (width 0.5) (layer "B.Cu") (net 12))
 (segment (start 144.525 102.775) (end 150.51 102.775) (width 0.5) (layer "B.Cu") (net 12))
 (segment (start 134.62 105.664) (end 134.62 104.1621) (width 0.5) (layer "B.Cu") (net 12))
 (segment (start 143.3884 103.9116) (end 144.525 102.775) (width 0.5) (layer "B.Cu") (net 12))
 (segment (start 136.9 97) (end 136.9424 97) (width 0.5) (layer "B.Cu") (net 12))
 (segment (start 134.62 103.9116) (end 143.3884 103.9116) (width 0.5) (layer "B.Cu") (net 12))
 (segment (start 136.9424 97) (end 142.3 91.6424) (width 0.5) (layer "B.Cu") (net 12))
 (segment (start 143.525 87.775) (end 148.96 87.775) (width 0.5) (layer "B.Cu") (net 12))
 (segment (start 137.16 104.34) (end 137.16 105.664) (width 0.5) (layer "F.Cu") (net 7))
 (segment (start 142.9 94.001284) (end 144 92.901284) (width 0.5) (layer "F.Cu") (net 7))
 (segment (start 139.23 102.27) (end 137.16 104.34) (width 0.5) (layer "F.Cu") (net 7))
 (segment (start 139.67 102.27) (end 139.67 101.6521) (width 0.5) (layer "F.Cu") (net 7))
 (segment (start 144 90.2) (end 144.425 89.775) (width 0.5) (layer "F.Cu") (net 7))
 (segment (start 150.51 105.275) (end 143.175 105.275) (width 0.5) (layer "F.Cu") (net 7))
 (segment (start 142.9 97.228) (end 142.9 94.001284) (width 0.5) (layer "F.Cu") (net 7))
 (segment (start 144 92.901284) (end 144 90.2) (width 0.5) (layer "F.Cu") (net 7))
 (segment (start 144.425 89.775) (end 148.96 89.775) (width 0.5) (layer "F.Cu") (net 7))
 (segment (start 139.67 102.27) (end 139.23 102.27) (width 0.5) (layer "F.Cu") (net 7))
 (segment (start 142.864 97.264) (end 142.9 97.228) (width 0.5) (layer "F.Cu") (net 7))
 (segment (start 143.175 105.275) (end 140.17 102.27) (width 0.5) (layer "F.Cu") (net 7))
 (segment (start 139.67 100.458) (end 139.67 101.6521) (width 0.5) (layer "F.Cu") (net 7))
 (segment (start 140.17 102.27) (end 139.67 102.27) (width 0.5) (layer "F.Cu") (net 7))
 (via (at 142.864 97.264) (size 0.8) (drill 0.4) (layers "F.Cu" "B.Cu") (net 7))
 (segment (start 142.864 97.264) (end 139.67 100.458) (width 0.5) (layer "B.Cu") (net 7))
 (segment (start 131.1 97.9) (end 132.05 98.85) (width 0.5) (layer "F.Cu") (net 10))
 (segment (start 132.05 98.85) (end 132.05 100.458) (width 0.5) (layer "F.Cu") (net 10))
 (segment (start 129.5 97.9) (end 131.1 97.9) (width 0.5) (layer "F.Cu") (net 10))
 (via (at 129.5 97.9) (size 0.8) (drill 0.4) (layers "F.Cu" "B.Cu") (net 10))
 (segment (start 143.2 92.3295) (end 143.2 90.1) (width 0.5) (layer "B.Cu") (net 10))
 (segment (start 125.8063 107.1747) (end 139.3253 107.1747) (width 0.5) (layer "B.Cu") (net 10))
 (segment (start 150.51 105.275) (end 141.5909 105.275) (width 0.5) (layer "B.Cu") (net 10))
 (segment (start 143.2 90.1) (end 143.525 89.775) (width 0.5) (layer "B.Cu") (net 10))
 (segment (start 136.7374 98.7921) (end 143.2 92.3295) (width 0.5) (layer "B.Cu") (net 10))
 (segment (start 127.3949 97.9) (end 125.4378 99.8571) (width 0.5) (layer "B.Cu") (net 10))
 (segment (start 133.7159 98.7921) (end 136.7374 98.7921) (width 0.5) (layer "B.Cu") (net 10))
 (segment (start 125.4378 106.8062) (end 125.8063 107.1747) (width 0.5) (layer "B.Cu") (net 10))
 (segment (start 139.7 106.8) (end 139.7 105.664) (width 0.5) (layer "B.Cu") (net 10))
 (segment (start 141.5909 105.275) (end 141.2019 105.664) (width 0.5) (layer "B.Cu") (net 10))
 (segment (start 125.4378 99.8571) (end 125.4378 106.8062) (width 0.5) (layer "B.Cu") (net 10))
 (segment (start 132.05 100.458) (end 133.7159 98.7921) (width 0.5) (layer "B.Cu") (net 10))
 (segment (start 129.5 97.9) (end 127.3949 97.9) (width 0.5) (layer "B.Cu") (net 10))
 (segment (start 139.3253 107.1747) (end 139.7 106.8) (width 0.5) (layer "B.Cu") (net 10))
 (segment (start 143.525 89.775) (end 148.96 89.775) (width 0.5) (layer "B.Cu") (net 10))
 (segment (start 139.7 105.664) (end 141.2019 105.664) (width 0.5) (layer "B.Cu") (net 10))
 (segment (start 134.59 88.5) (end 134.59 90.298) (width 0.5) (layer "F.Cu") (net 3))
 (segment (start 135.89 85.852) (end 135.89 87.2) (width 0.5) (layer "F.Cu") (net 3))
 (segment (start 135.89 87.2) (end 134.59 88.5) (width 0.5) (layer "F.Cu") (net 3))
 (segment (start 134.5869 88.4969) (end 134.59 88.5) (width 0.5) (layer "F.Cu") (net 3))
 (segment (start 83.06 86.995) (end 83.06 88.14) (width 0.5) (layer "F.Cu") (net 3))
 (segment (start 83.06 88.14) (end 83.4169 88.4969) (width 0.5) (layer "F.Cu") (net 3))
 (segment (start 83.4169 88.4969) (end 134.5869 88.4969) (width 0.5) (layer "F.Cu") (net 3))
 (segment (start 141.2221 91.37) (end 139.3006 93.2915) (width 0.5) (layer "F.Cu") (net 9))
 (segment (start 133.35 85.852) (end 133.35 84.65) (width 0.5) (layer "F.Cu") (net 9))
 (segment (start 137.081 84.3501) (end 141.2221 88.4912) (width 0.5) (layer "F.Cu") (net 9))
 (segment (start 134.59 100.458) (end 134.59 97.6813) (width 0.5) (layer "F.Cu") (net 9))
 (segment (start 139.3006 93.2915) (end 138.6694 93.2915) (width 0.5) (layer "F.Cu") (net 9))
 (segment (start 133.35 84.65) (end 133.6499 84.3501) (width 0.5) (layer "F.Cu") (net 9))
 (segment (start 133.6499 84.3501) (end 137.081 84.3501) (width 0.5) (layer "F.Cu") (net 9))
 (segment (start 141.2221 88.4912) (end 141.2221 91.37) (width 0.5) (layer "F.Cu") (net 9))
 (via (at 138.6694 93.2915) (size 0.8) (drill 0.4) (layers "F.Cu" "B.Cu") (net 9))
 (via (at 134.59 97.6813) (size 0.8) (drill 0.4) (layers "F.Cu" "B.Cu") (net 9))
 (segment (start 138.6694 93.2915) (end 134.59 97.3709) (width 0.5) (layer "B.Cu") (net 9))
 (segment (start 134.59 97.3709) (end 134.59 97.6813) (width 0.5) (layer "B.Cu") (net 9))
 (segment (start 73.2711 85.4789) (end 128.935 85.4789) (width 0.5) (layer "B.Cu") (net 13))
 (segment (start 72.9 85.85) (end 73.2711 85.4789) (width 0.5) (layer "B.Cu") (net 13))
 (segment (start 72.9 86.995) (end 72.9 85.85) (width 0.5) (layer "B.Cu") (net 13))
 (segment (start 128.935 85.4789) (end 129.3081 85.852) (width 0.5) (layer "B.Cu") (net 13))
 (segment (start 129.3081 85.852) (end 130.81 85.852) (width 0.5) (layer "B.Cu") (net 13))
 (segment (start 126.511608 94.6156) (end 135.7624 94.6156) (width 0.5) (layer "F.Cu") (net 1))
 (segment (start 135.7624 94.6156) (end 138.176 92.202) (width 0.5) (layer "F.Cu") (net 1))
 (segment (start 72.9 102.868) (end 73.406 102.362) (width 0.5) (layer "F.Cu") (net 1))
 (segment (start 124.5576 96.569608) (end 126.511608 94.6156) (width 0.5) (layer "F.Cu") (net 1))
 (segment (start 123.952 102.362) (end 124.5576 101.7564) (width 0.5) (layer "F.Cu") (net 1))
 (segment (start 72.9 104.775) (end 72.9 102.868) (width 0.5) (layer "F.Cu") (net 1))
 (segment (start 138.176 92.202) (end 139.117308 92.202) (width 0.5) (layer "F.Cu") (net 1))
 (segment (start 139.117308 92.202) (end 139.67 91.649308) (width 0.5) (layer "F.Cu") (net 1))
 (segment (start 73.406 102.362) (end 123.952 102.362) (width 0.5) (layer "F.Cu") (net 1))
 (segment (start 124.5576 101.7564) (end 124.5576 96.569608) (width 0.5) (layer "F.Cu") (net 1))
 (segment (start 139.67 91.649308) (end 139.67 90.298) (width 0.5) (layer "F.Cu") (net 1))
 (segment (start 123.79 99.21) (end 126.5 96.5) (width 0.5) (layer "B.Cu") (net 2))
 (segment (start 132.3 96.5) (end 137.13 91.67) (width 0.5) (layer "B.Cu") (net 2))
 (segment (start 122.2731 106.2769) (end 123.79 104.76) (width 0.5) (layer "B.Cu") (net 2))
 (segment (start 75.8769 106.2769) (end 122.2731 106.2769) (width 0.5) (layer "B.Cu") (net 2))
 (segment (start 75.44 104.775) (end 75.44 105.84) (width 0.5) (layer "B.Cu") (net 2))
 (segment (start 126.5 96.5) (end 132.3 96.5) (width 0.5) (layer "B.Cu") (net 2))
 (segment (start 137.13 91.67) (end 137.13 90.298) (width 0.5) (layer "B.Cu") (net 2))
 (segment (start 123.79 104.76) (end 123.79 99.21) (width 0.5) (layer "B.Cu") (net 2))
 (segment (start 75.44 105.84) (end 75.8769 106.2769) (width 0.5) (layer "B.Cu") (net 2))
 (segment (start 90.68 104.775) (end 90.68 103.67) (width 0.5) (layer "F.Cu") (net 4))
 (segment (start 90.68 103.67) (end 90.2831 103.2731) (width 0.5) (layer "F.Cu") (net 4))
 (segment (start 78.4269 103.2731) (end 77.98 103.72) (width 0.5) (layer "F.Cu") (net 4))
 (segment (start 90.2831 103.2731) (end 78.4269 103.2731) (width 0.5) (layer "F.Cu") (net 4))
 (segment (start 77.98 103.72) (end 77.98 104.775) (width 0.5) (layer "F.Cu") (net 4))
 (segment (start 123.3031 88.4969) (end 123.9925 87.8075) (width 0.5) (layer "B.Cu") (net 4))
 (segment (start 116.0785 88.4969) (end 116.08 88.4954) (width 0.5) (layer "B.Cu") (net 4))
 (segment (start 103.38 88.4969) (end 116.0785 88.4969) (width 0.5) (layer "B.Cu") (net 4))
 (segment (start 90.68 88.4969) (end 103.38 88.4969) (width 0.5) (layer "B.Cu") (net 4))
 (segment (start 103.38 86.995) (end 103.38 88.4969) (width 0.5) (layer "B.Cu") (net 4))
 (segment (start 90.68 104.775) (end 92.18 103.275) (width 0.5) (layer "B.Cu") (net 4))
 (segment (start 116.08 88.4117) (end 116.08 88.4954) (width 0.5) (layer "B.Cu") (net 4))
 (segment (start 115.645 103.275) (end 103.3819 103.275) (width 0.5) (layer "B.Cu") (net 4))
 (segment (start 77.98 86.995) (end 77.98 88.4969) (width 0.5) (layer "B.Cu") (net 4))
 (segment (start 77.98 88.4969) (end 77.98 103.2731) (width 0.5) (layer "B.Cu") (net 4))
 (segment (start 130.9075 87.8075) (end 132.05 88.95) (width 0.5) (layer "B.Cu") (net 4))
 (segment (start 116.08 86.995) (end 116.08 88.4117) (width 0.5) (layer "B.Cu") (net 4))
 (segment (start 103.38 103.2769) (end 103.38 104.775) (width 0.5) (layer "B.Cu") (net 4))
 (segment (start 103.3819 103.275) (end 103.38 103.2769) (width 0.5) (layer "B.Cu") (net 4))
 (segment (start 123.9925 87.8075) (end 130.9075 87.8075) (width 0.5) (layer "B.Cu") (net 4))
 (segment (start 132.05 88.95) (end 132.05 90.298) (width 0.5) (layer "B.Cu") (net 4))
 (segment (start 77.98 104.775) (end 77.98 103.2731) (width 0.5) (layer "B.Cu") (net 4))
 (segment (start 116.0815 88.4969) (end 123.3031 88.4969) (width 0.5) (layer "B.Cu") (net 4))
 (segment (start 92.18 103.275) (end 103.3819 103.275) (width 0.5) (layer "B.Cu") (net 4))
 (segment (start 77.98 88.4969) (end 90.68 88.4969) (width 0.5) (layer "B.Cu") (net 4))
 (segment (start 116.08 103.71) (end 115.645 103.275) (width 0.5) (layer "B.Cu") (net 4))
 (segment (start 116.08 88.4954) (end 116.0815 88.4969) (width 0.5) (layer "B.Cu") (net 4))
 (segment (start 116.08 104.775) (end 116.08 103.71) (width 0.5) (layer "B.Cu") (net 4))
 (segment (start 90.68 88.4969) (end 90.68 86.995) (width 0.5) (layer "B.Cu") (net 4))
 (segment (start 80.52 102.87) (end 80.52 104.775) (width 0.5) (layer "B.Cu") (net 5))
 (segment (start 129.51 90.298) (end 129.51 89.31) (width 0.5) (layer "B.Cu") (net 5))
 (segment (start 112.7968 101.3032) (end 82.0868 101.3032) (width 0.5) (layer "B.Cu") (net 5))
 (segment (start 128.9782 88.7782) (end 125.3218 88.7782) (width 0.5) (layer "B.Cu") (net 5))
 (segment (start 82.0868 101.3032) (end 80.52 102.87) (width 0.5) (layer "B.Cu") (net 5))
 (segment (start 129.51 89.31) (end 128.9782 88.7782) (width 0.5) (layer "B.Cu") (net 5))
 (segment (start 125.3218 88.7782) (end 112.7968 101.3032) (width 0.5) (layer "B.Cu") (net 5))
 (segment (start 83.06 103.15) (end 83.9355 102.2745) (width 0.5) (layer "B.Cu") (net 6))
 (segment (start 118.2255 102.2745) (end 126.97 93.53) (width 0.5) (layer "B.Cu") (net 6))
 (segment (start 83.9355 102.2745) (end 118.2255 102.2745) (width 0.5) (layer "B.Cu") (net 6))
 (segment (start 126.97 93.53) (end 126.97 90.298) (width 0.5) (layer "B.Cu") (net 6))
 (segment (start 83.06 104.775) (end 83.06 103.15) (width 0.5) (layer "B.Cu") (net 6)))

